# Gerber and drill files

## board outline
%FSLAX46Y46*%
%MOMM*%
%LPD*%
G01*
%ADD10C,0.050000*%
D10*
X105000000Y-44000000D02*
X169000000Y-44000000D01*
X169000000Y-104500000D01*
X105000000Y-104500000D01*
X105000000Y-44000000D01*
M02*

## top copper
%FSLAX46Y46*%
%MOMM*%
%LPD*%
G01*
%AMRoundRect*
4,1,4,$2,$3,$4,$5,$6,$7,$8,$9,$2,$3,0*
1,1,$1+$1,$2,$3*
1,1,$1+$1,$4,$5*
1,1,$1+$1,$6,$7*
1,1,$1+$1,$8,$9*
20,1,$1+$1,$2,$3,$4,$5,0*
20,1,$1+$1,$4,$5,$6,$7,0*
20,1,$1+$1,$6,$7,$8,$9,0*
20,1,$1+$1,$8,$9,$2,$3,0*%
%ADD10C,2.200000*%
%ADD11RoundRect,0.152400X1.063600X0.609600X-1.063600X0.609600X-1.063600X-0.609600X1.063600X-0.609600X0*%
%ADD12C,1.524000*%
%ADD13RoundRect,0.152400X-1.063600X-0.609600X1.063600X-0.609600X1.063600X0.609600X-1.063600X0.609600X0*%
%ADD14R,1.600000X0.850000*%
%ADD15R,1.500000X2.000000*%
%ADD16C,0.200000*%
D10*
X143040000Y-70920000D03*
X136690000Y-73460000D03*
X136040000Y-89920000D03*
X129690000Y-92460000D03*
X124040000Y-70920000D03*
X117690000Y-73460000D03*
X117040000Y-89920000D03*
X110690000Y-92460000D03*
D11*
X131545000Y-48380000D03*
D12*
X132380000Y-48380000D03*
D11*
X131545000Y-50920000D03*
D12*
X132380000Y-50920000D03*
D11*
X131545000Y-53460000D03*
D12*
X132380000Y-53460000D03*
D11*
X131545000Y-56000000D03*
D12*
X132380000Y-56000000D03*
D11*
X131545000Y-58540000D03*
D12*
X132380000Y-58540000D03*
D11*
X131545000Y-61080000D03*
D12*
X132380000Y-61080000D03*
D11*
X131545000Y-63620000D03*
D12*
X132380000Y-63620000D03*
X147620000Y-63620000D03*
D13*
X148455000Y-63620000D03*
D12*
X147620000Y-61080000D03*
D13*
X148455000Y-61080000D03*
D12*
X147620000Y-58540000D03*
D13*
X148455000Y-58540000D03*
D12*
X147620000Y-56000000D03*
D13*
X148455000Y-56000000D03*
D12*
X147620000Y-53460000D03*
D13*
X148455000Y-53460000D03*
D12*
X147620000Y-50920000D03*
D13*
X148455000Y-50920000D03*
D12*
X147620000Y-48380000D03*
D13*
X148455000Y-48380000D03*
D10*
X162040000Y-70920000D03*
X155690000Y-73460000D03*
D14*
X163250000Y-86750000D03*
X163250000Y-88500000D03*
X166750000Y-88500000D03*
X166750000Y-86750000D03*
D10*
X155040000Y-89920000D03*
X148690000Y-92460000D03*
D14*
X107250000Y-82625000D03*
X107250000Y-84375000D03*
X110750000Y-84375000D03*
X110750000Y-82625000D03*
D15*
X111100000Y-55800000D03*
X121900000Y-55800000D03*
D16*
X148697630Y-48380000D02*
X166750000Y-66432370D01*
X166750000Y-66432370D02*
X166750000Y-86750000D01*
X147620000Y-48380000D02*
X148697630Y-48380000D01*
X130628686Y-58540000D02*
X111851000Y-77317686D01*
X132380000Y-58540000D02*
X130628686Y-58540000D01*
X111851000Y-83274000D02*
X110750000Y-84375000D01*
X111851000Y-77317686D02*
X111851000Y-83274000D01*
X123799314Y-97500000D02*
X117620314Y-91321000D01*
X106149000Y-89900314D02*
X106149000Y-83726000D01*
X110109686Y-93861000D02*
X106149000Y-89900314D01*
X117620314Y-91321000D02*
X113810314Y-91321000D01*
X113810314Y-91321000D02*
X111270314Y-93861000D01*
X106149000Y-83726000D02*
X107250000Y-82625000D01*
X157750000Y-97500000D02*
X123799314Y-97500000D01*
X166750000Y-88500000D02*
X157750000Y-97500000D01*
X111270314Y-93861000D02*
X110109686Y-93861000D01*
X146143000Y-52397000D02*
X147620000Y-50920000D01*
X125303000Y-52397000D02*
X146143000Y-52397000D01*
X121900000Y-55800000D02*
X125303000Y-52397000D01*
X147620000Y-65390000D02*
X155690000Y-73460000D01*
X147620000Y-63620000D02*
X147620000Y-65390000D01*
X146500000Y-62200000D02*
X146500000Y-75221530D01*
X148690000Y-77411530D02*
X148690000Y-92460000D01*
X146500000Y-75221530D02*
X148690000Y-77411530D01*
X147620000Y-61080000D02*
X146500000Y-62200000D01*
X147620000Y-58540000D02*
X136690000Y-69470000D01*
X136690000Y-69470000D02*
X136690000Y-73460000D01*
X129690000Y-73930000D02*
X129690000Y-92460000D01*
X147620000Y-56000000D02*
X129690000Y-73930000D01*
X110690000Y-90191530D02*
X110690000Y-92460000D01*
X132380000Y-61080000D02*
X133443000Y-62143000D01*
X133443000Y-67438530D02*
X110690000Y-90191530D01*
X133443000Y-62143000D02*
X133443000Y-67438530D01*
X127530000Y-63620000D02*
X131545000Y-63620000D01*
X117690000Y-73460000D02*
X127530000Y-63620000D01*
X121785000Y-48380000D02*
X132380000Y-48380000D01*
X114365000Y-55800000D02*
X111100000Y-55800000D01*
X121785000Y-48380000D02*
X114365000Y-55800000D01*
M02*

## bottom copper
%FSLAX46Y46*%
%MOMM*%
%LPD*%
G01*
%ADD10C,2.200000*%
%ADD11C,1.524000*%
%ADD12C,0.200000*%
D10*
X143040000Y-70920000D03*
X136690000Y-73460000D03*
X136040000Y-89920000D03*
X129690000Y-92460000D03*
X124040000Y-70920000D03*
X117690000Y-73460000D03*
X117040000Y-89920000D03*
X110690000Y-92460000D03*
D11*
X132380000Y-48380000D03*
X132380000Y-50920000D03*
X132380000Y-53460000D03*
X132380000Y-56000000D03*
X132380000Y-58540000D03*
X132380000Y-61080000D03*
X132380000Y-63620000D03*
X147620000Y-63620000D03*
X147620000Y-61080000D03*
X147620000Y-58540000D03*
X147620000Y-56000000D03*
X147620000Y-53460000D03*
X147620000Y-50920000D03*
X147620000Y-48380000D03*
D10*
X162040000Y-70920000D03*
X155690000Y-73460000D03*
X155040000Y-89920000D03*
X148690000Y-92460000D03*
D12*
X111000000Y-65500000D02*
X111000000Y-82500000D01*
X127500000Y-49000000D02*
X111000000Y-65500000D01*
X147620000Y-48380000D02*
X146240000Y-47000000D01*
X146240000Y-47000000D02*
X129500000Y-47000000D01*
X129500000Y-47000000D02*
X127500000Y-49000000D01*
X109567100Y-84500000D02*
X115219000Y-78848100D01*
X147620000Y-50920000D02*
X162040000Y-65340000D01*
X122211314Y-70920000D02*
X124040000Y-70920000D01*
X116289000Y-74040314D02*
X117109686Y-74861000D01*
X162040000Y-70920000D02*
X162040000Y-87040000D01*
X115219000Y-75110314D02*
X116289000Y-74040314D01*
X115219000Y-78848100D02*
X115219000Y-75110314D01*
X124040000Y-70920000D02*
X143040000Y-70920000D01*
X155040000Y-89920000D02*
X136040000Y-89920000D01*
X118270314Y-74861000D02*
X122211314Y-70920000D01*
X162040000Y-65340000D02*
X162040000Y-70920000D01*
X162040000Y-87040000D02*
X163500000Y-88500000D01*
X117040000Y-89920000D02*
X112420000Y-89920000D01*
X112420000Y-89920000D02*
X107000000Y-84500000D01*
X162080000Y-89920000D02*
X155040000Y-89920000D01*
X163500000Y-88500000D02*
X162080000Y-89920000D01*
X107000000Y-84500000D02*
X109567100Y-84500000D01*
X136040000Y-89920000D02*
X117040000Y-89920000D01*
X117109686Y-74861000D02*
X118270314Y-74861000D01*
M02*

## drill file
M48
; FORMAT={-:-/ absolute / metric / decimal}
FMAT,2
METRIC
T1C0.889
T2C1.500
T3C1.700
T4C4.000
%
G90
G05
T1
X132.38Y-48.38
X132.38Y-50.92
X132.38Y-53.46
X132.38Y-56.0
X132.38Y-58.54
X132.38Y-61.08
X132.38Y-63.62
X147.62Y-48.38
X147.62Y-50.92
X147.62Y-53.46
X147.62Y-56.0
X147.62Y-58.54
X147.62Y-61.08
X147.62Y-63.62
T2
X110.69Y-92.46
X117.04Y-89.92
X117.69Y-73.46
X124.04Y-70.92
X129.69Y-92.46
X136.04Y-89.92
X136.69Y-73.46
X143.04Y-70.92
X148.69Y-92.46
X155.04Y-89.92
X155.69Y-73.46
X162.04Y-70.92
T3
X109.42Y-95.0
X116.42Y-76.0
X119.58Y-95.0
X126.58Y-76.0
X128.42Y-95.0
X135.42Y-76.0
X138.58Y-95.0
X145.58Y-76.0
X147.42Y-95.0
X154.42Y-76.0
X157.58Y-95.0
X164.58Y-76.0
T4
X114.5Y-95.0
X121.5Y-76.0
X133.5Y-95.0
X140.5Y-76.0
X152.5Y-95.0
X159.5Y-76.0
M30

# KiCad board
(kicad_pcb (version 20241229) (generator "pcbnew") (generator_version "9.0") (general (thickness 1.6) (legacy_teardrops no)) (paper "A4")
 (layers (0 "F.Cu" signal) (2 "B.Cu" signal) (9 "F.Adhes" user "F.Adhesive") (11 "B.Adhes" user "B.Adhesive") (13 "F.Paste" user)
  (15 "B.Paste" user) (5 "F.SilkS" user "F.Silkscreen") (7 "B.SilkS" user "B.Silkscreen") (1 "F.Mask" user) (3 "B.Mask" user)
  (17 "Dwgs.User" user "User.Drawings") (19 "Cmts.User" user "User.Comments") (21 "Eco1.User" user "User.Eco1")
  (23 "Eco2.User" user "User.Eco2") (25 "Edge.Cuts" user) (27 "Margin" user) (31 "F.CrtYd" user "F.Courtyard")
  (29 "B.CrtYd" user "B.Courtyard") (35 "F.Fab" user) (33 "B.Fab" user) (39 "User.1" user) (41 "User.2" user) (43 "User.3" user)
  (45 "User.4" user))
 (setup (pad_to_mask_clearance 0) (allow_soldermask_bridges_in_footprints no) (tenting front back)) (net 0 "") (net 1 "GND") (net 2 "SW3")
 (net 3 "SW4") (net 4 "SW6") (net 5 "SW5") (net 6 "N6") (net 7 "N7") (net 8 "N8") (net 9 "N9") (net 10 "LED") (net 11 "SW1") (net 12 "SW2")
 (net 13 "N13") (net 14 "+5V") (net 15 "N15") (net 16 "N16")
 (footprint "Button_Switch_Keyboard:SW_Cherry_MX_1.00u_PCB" (layer "F.Cu") (at 143.04 70.92)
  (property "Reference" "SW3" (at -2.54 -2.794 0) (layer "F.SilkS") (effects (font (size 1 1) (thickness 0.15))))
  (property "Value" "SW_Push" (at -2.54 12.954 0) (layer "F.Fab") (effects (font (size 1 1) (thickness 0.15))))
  (pad "" np_thru_hole circle (at -7.62 5.08) (size 1.7 1.7) (drill 1.7) (layers "*.Cu" "*.Mask"))
  (pad "" np_thru_hole circle (at -2.54 5.08) (size 4 4) (drill 4) (layers "*.Cu" "*.Mask"))
  (pad "" np_thru_hole circle (at 2.54 5.08) (size 1.7 1.7) (drill 1.7) (layers "*.Cu" "*.Mask"))
  (pad "1" thru_hole circle (at 0 0) (size 2.2 2.2) (drill 1.5) (layers "*.Cu" "*.Mask") (remove_unused_layers no) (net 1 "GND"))
  (pad "2" thru_hole circle (at -6.35 2.54) (size 2.2 2.2) (drill 1.5) (layers "*.Cu" "*.Mask") (remove_unused_layers no) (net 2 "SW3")))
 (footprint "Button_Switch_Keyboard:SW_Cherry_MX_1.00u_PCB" (layer "F.Cu") (at 136.04 89.92)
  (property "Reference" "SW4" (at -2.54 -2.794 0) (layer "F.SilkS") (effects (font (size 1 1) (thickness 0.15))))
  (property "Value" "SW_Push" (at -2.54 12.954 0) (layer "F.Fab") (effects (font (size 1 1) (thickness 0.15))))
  (pad "" np_thru_hole circle (at -7.62 5.08) (size 1.7 1.7) (drill 1.7) (layers "*.Cu" "*.Mask"))
  (pad "" np_thru_hole circle (at -2.54 5.08) (size 4 4) (drill 4) (layers "*.Cu" "*.Mask"))
  (pad "" np_thru_hole circle (at 2.54 5.08) (size 1.7 1.7) (drill 1.7) (layers "*.Cu" "*.Mask"))
  (pad "1" thru_hole circle (at 0 0) (size 2.2 2.2) (drill 1.5) (layers "*.Cu" "*.Mask") (remove_unused_layers no) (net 1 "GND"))
  (pad "2" thru_hole circle (at -6.35 2.54) (size 2.2 2.2) (drill 1.5) (layers "*.Cu" "*.Mask") (remove_unused_layers no) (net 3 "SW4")))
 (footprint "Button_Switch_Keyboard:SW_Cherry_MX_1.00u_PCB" (layer "F.Cu") (at 124.04 70.92)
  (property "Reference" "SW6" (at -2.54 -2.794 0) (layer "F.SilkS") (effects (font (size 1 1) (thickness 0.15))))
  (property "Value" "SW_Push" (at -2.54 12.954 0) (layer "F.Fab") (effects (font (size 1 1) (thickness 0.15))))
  (pad "" np_thru_hole circle (at -7.62 5.08) (size 1.7 1.7) (drill 1.7) (layers "*.Cu" "*.Mask"))
  (pad "" np_thru_hole circle (at -2.54 5.08) (size 4 4) (drill 4) (layers "*.Cu" "*.Mask"))
  (pad "" np_thru_hole circle (at 2.54 5.08) (size 1.7 1.7) (drill 1.7) (layers "*.Cu" "*.Mask"))
  (pad "1" thru_hole circle (at 0 0) (size 2.2 2.2) (drill 1.5) (layers "*.Cu" "*.Mask") (remove_unused_layers no) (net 1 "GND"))
  (pad "2" thru_hole circle (at -6.35 2.54) (size 2.2 2.2) (drill 1.5) (layers "*.Cu" "*.Mask") (remove_unused_layers no) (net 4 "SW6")))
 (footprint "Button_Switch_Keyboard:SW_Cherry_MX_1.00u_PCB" (layer "F.Cu") (at 117.04 89.92)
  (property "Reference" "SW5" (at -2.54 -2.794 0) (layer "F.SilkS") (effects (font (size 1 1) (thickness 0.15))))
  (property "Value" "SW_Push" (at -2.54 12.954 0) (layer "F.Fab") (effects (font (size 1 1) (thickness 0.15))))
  (pad "" np_thru_hole circle (at -7.62 5.08) (size 1.7 1.7) (drill 1.7) (layers "*.Cu" "*.Mask"))
  (pad "" np_thru_hole circle (at -2.54 5.08) (size 4 4) (drill 4) (layers "*.Cu" "*.Mask"))
  (pad "" np_thru_hole circle (at 2.54 5.08) (size 1.7 1.7) (drill 1.7) (layers "*.Cu" "*.Mask"))
  (pad "1" thru_hole circle (at 0 0) (size 2.2 2.2) (drill 1.5) (layers "*.Cu" "*.Mask") (remove_unused_layers no) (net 1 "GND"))
  (pad "2" thru_hole circle (at -6.35 2.54) (size 2.2 2.2) (drill 1.5) (layers "*.Cu" "*.Mask") (remove_unused_layers no) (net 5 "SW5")))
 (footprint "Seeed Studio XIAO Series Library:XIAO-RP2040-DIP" (layer "F.Cu") (at 140 56)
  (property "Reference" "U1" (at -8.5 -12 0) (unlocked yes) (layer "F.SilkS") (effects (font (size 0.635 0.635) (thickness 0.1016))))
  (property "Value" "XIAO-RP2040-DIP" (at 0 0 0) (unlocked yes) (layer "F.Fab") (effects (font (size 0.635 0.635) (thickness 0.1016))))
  (pad "1" smd roundrect (at -8.455 -7.62 180) (size 2.432 1.524) (layers "F.Cu" "F.Mask") (roundrect_rratio 0.1) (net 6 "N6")
   (thermal_bridge_angle 45))
  (pad "1" thru_hole circle (at -7.62 -7.62 180) (size 1.524 1.524) (drill 0.889) (layers "*.Cu" "*.Mask") (remove_unused_layers no)
   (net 6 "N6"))
  (pad "2" smd roundrect (at -8.455 -5.08 180) (size 2.432 1.524) (layers "F.Cu" "F.Mask") (roundrect_rratio 0.1) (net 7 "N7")
   (thermal_bridge_angle 45))
  (pad "2" thru_hole circle (at -7.62 -5.08 180) (size 1.524 1.524) (drill 0.889) (layers "*.Cu" "*.Mask") (remove_unused_layers no)
   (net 7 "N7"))
  (pad "3" smd roundrect (at -8.455 -2.54 180) (size 2.432 1.524) (layers "F.Cu" "F.Mask") (roundrect_rratio 0.1) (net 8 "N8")
   (thermal_bridge_angle 45))
  (pad "3" thru_hole circle (at -7.62 -2.54 180) (size 1.524 1.524) (drill 0.889) (layers "*.Cu" "*.Mask") (remove_unused_layers no)
   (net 8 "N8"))
  (pad "4" smd roundrect (at -8.455 0 180) (size 2.432 1.524) (layers "F.Cu" "F.Mask") (roundrect_rratio 0.1) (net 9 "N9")
   (thermal_bridge_angle 45))
  (pad "4" thru_hole circle (at -7.62 0 180) (size 1.524 1.524) (drill 0.889) (layers "*.Cu" "*.Mask") (remove_unused_layers no)
   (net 9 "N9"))
  (pad "5" smd roundrect (at -8.455 2.54 180) (size 2.432 1.524) (layers "F.Cu" "F.Mask") (roundrect_rratio 0.1) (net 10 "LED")
   (thermal_bridge_angle 45))
  (pad "5" thru_hole circle (at -7.62 2.54 180) (size 1.524 1.524) (drill 0.889) (layers "*.Cu" "*.Mask") (remove_unused_layers no)
   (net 10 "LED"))
  (pad "6" smd roundrect (at -8.455 5.08 180) (size 2.432 1.524) (layers "F.Cu" "F.Mask") (roundrect_rratio 0.1) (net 5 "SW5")
   (thermal_bridge_angle 45))
  (pad "6" thru_hole circle (at -7.62 5.08 180) (size 1.524 1.524) (drill 0.889) (layers "*.Cu" "*.Mask") (remove_unused_layers no)
   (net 5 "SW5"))
  (pad "7" smd roundrect (at -8.455 7.62 180) (size 2.432 1.524) (layers "F.Cu" "F.Mask") (roundrect_rratio 0.1) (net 4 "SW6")
   (thermal_bridge_angle 45))
  (pad "7" thru_hole circle (at -7.62 7.62 180) (size 1.524 1.524) (drill 0.889) (layers "*.Cu" "*.Mask") (remove_unused_layers no)
   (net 4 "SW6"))
  (pad "8" thru_hole circle (at 7.62 7.62) (size 1.524 1.524) (drill 0.889) (layers "*.Cu" "*.Mask") (remove_unused_layers no)
   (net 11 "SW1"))
  (pad "8" smd roundrect (at 8.455 7.62) (size 2.432 1.524) (layers "F.Cu" "F.Mask") (roundrect_rratio 0.1) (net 11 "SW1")
   (thermal_bridge_angle 45))
  (pad "9" thru_hole circle (at 7.62 5.08) (size 1.524 1.524) (drill 0.889) (layers "*.Cu" "*.Mask") (remove_unused_layers no)
   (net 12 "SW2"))
  (pad "9" smd roundrect (at 8.455 5.08) (size 2.432 1.524) (layers "F.Cu" "F.Mask") (roundrect_rratio 0.1) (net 12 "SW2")
   (thermal_bridge_angle 45))
  (pad "10" thru_hole circle (at 7.62 2.54) (size 1.524 1.524) (drill 0.889) (layers "*.Cu" "*.Mask") (remove_unused_layers no)
   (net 2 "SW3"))
  (pad "10" smd roundrect (at 8.455 2.54) (size 2.432 1.524) (layers "F.Cu" "F.Mask") (roundrect_rratio 0.1) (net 2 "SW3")
   (thermal_bridge_angle 45))
  (pad "11" thru_hole circle (at 7.62 0) (size 1.524 1.524) (drill 0.889) (layers "*.Cu" "*.Mask") (remove_unused_layers no) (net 3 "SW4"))
  (pad "11" smd roundrect (at 8.455 0) (size 2.432 1.524) (layers "F.Cu" "F.Mask") (roundrect_rratio 0.1) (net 3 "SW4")
   (thermal_bridge_angle 45))
  (pad "12" thru_hole circle (at 7.62 -2.54) (size 1.524 1.524) (drill 0.889) (layers "*.Cu" "*.Mask") (remove_unused_layers no)
   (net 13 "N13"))
  (pad "12" smd roundrect (at 8.455 -2.54) (size 2.432 1.524) (layers "F.Cu" "F.Mask") (roundrect_rratio 0.1) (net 13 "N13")
   (thermal_bridge_angle 45))
  (pad "13" thru_hole circle (at 7.62 -5.08) (size 1.524 1.524) (drill 0.889) (layers "*.Cu" "*.Mask") (remove_unused_layers no)
   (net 1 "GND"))
  (pad "13" smd roundrect (at 8.455 -5.08) (size 2.432 1.524) (layers "F.Cu" "F.Mask") (roundrect_rratio 0.1) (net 1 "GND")
   (thermal_bridge_angle 45))
  (pad "14" thru_hole circle (at 7.62 -7.62) (size 1.524 1.524) (drill 0.889) (layers "*.Cu" "*.Mask") (remove_unused_layers no)
   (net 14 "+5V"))
  (pad "14" smd roundrect (at 8.455 -7.62) (size 2.432 1.524) (layers "F.Cu" "F.Mask") (roundrect_rratio 0.1) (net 14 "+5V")
   (thermal_bridge_angle 45)))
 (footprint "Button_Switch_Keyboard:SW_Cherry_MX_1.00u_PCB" (layer "F.Cu") (at 162.04 70.92)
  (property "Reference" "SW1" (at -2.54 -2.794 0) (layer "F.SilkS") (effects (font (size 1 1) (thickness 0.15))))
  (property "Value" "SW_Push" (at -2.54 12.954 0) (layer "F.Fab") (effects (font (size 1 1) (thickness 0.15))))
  (pad "" np_thru_hole circle (at -7.62 5.08) (size 1.7 1.7) (drill 1.7) (layers "*.Cu" "*.Mask"))
  (pad "" np_thru_hole circle (at -2.54 5.08) (size 4 4) (drill 4) (layers "*.Cu" "*.Mask"))
  (pad "" np_thru_hole circle (at 2.54 5.08) (size 1.7 1.7) (drill 1.7) (layers "*.Cu" "*.Mask"))
  (pad "1" thru_hole circle (at 0 0) (size 2.2 2.2) (drill 1.5) (layers "*.Cu" "*.Mask") (remove_unused_layers no) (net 1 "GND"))
  (pad "2" thru_hole circle (at -6.35 2.54) (size 2.2 2.2) (drill 1.5) (layers "*.Cu" "*.Mask") (remove_unused_layers no) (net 11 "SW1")))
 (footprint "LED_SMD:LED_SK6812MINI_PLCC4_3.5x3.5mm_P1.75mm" (layer "F.Cu") (at 165 87.625)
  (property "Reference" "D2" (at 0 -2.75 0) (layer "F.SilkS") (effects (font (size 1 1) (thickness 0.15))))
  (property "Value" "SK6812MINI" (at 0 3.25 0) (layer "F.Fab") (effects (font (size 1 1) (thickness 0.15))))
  (pad "1" smd rect (at -1.75 -0.875) (size 1.6 0.85) (layers "F.Cu" "F.Mask" "F.Paste") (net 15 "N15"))
  (pad "2" smd rect (at -1.75 0.875) (size 1.6 0.85) (layers "F.Cu" "F.Mask" "F.Paste") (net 1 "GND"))
  (pad "3" smd rect (at 1.75 0.875) (size 1.6 0.85) (layers "F.Cu" "F.Mask" "F.Paste") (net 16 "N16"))
  (pad "4" smd rect (at 1.75 -0.875) (size 1.6 0.85) (layers "F.Cu" "F.Mask" "F.Paste") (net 14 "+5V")))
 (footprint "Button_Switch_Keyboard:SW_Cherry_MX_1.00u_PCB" (layer "F.Cu") (at 155.04 89.92)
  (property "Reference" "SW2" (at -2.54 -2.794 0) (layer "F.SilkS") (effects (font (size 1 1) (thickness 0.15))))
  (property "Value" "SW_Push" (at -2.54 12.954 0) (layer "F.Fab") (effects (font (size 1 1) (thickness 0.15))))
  (pad "" np_thru_hole circle (at -7.62 5.08) (size 1.7 1.7) (drill 1.7) (layers "*.Cu" "*.Mask"))
  (pad "" np_thru_hole circle (at -2.54 5.08) (size 4 4) (drill 4) (layers "*.Cu" "*.Mask"))
  (pad "" np_thru_hole circle (at 2.54 5.08) (size 1.7 1.7) (drill 1.7) (layers "*.Cu" "*.Mask"))
  (pad "1" thru_hole circle (at 0 0) (size 2.2 2.2) (drill 1.5) (layers "*.Cu" "*.Mask") (remove_unused_layers no) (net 1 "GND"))
  (pad "2" thru_hole circle (at -6.35 2.54) (size 2.2 2.2) (drill 1.5) (layers "*.Cu" "*.Mask") (remove_unused_layers no) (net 12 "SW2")))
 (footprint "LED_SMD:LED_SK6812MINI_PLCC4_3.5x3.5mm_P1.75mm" (layer "F.Cu") (at 109 83.5)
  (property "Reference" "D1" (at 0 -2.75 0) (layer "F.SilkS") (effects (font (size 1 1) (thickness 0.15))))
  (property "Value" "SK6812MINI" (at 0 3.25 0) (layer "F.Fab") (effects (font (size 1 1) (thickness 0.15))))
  (pad "1" smd rect (at -1.75 -0.875) (size 1.6 0.85) (layers "F.Cu" "F.Mask" "F.Paste") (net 16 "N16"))
  (pad "2" smd rect (at -1.75 0.875) (size 1.6 0.85) (layers "F.Cu" "F.Mask" "F.Paste") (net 1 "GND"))
  (pad "3" smd rect (at 1.75 0.875) (size 1.6 0.85) (layers "F.Cu" "F.Mask" "F.Paste") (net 10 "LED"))
  (pad "4" smd rect (at 1.75 -0.875) (size 1.6 0.85) (layers "F.Cu" "F.Mask" "F.Paste") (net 14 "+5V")))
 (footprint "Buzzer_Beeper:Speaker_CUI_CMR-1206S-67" (layer "F.Cu") (at 116.5 53.5)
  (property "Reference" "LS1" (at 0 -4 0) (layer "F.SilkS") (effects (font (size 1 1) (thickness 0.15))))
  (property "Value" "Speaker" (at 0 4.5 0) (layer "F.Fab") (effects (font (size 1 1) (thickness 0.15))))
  (pad "1" smd rect (at -5.4 2.3 180) (size 1.5 2) (layers "F.Cu" "F.Mask") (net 6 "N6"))
  (pad "2" smd rect (at 5.4 2.3 180) (size 1.5 2) (layers "F.Cu" "F.Mask") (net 1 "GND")))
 (gr_rect (start 105 44) (end 169 104.5) (stroke (width 0.05) (type default)) (fill no) (layer "Edge.Cuts"))
 (segment (start 148.69763 48.38) (end 166.75 66.43237) (width 0.2) (layer "F.Cu") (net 14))
 (segment (start 166.75 66.43237) (end 166.75 86.75) (width 0.2) (layer "F.Cu") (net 14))
 (segment (start 147.62 48.38) (end 148.69763 48.38) (width 0.2) (layer "F.Cu") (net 14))
 (segment (start 111 65.5) (end 111 82.5) (width 0.2) (layer "B.Cu") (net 14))
 (segment (start 127.5 49) (end 111 65.5) (width 0.2) (layer "B.Cu") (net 14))
 (segment (start 147.62 48.38) (end 146.24 47) (width 0.2) (layer "B.Cu") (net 14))
 (segment (start 146.24 47) (end 129.5 47) (width 0.2) (layer "B.Cu") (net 14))
 (segment (start 129.5 47) (end 127.5 49) (width 0.2) (layer "B.Cu") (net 14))
 (segment (start 130.628686 58.54) (end 111.851 77.317686) (width 0.2) (layer "F.Cu") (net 10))
 (segment (start 132.38 58.54) (end 130.628686 58.54) (width 0.2) (layer "F.Cu") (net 10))
 (segment (start 111.851 83.274) (end 110.75 84.375) (width 0.2) (layer "F.Cu") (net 10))
 (segment (start 111.851 77.317686) (end 111.851 83.274) (width 0.2) (layer "F.Cu") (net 10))
 (segment (start 123.799314 97.5) (end 117.620314 91.321) (width 0.2) (layer "F.Cu") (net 16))
 (segment (start 106.149 89.900314) (end 106.149 83.726) (width 0.2) (layer "F.Cu") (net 16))
 (segment (start 110.109686 93.861) (end 106.149 89.900314) (width 0.2) (layer "F.Cu") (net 16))
 (segment (start 117.620314 91.321) (end 113.810314 91.321) (width 0.2) (layer "F.Cu") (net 16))
 (segment (start 113.810314 91.321) (end 111.270314 93.861) (width 0.2) (layer "F.Cu") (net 16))
 (segment (start 106.149 83.726) (end 107.25 82.625) (width 0.2) (layer "F.Cu") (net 16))
 (segment (start 157.75 97.5) (end 123.799314 97.5) (width 0.2) (layer "F.Cu") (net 16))
 (segment (start 166.75 88.5) (end 157.75 97.5) (width 0.2) (layer "F.Cu") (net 16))
 (segment (start 111.270314 93.861) (end 110.109686 93.861) (width 0.2) (layer "F.Cu") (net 16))
 (segment (start 146.143 52.397) (end 147.62 50.92) (width 0.2) (layer "F.Cu") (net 1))
 (segment (start 125.303 52.397) (end 146.143 52.397) (width 0.2) (layer "F.Cu") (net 1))
 (segment (start 121.9 55.8) (end 125.303 52.397) (width 0.2) (layer "F.Cu") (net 1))
 (segment (start 109.5671 84.5) (end 115.219 78.8481) (width 0.2) (layer "B.Cu") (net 1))
 (segment (start 147.62 50.92) (end 162.04 65.34) (width 0.2) (layer "B.Cu") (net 1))
 (segment (start 122.211314 70.92) (end 124.04 70.92) (width 0.2) (layer "B.Cu") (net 1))
 (segment (start 116.289 74.040314) (end 117.109686 74.861) (width 0.2) (layer "B.Cu") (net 1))
 (segment (start 162.04 70.92) (end 162.04 87.04) (width 0.2) (layer "B.Cu") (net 1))
 (segment (start 115.219 75.110314) (end 116.289 74.040314) (width 0.2) (layer "B.Cu") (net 1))
 (segment (start 115.219 78.8481) (end 115.219 75.110314) (width 0.2) (layer "B.Cu") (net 1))
 (segment (start 124.04 70.92) (end 143.04 70.92) (width 0.2) (layer "B.Cu") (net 1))
 (segment (start 155.04 89.92) (end 136.04 89.92) (width 0.2) (layer "B.Cu") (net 1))
 (segment (start 118.270314 74.861) (end 122.211314 70.92) (width 0.2) (layer "B.Cu") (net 1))
 (segment (start 162.04 65.34) (end 162.04 70.92) (width 0.2) (layer "B.Cu") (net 1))
 (segment (start 162.04 87.04) (end 163.5 88.5) (width 0.2) (layer "B.Cu") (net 1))
 (segment (start 117.04 89.92) (end 112.42 89.92) (width 0.2) (layer "B.Cu") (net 1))
 (segment (start 112.42 89.92) (end 107 84.5) (width 0.2) (layer "B.Cu") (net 1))
 (segment (start 162.08 89.92) (end 155.04 89.92) (width 0.2) (layer "B.Cu") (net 1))
 (segment (start 163.5 88.5) (end 162.08 89.92) (width 0.2) (layer "B.Cu") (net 1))
 (segment (start 107 84.5) (end 109.5671 84.5) (width 0.2) (layer "B.Cu") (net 1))
 (segment (start 136.04 89.92) (end 117.04 89.92) (width 0.2) (layer "B.Cu") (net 1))
 (segment (start 117.109686 74.861) (end 118.270314 74.861) (width 0.2) (layer "B.Cu") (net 1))
 (segment (start 147.62 65.39) (end 155.69 73.46) (width 0.2) (layer "F.Cu") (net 11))
 (segment (start 147.62 63.62) (end 147.62 65.39) (width 0.2) (layer "F.Cu") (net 11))
 (segment (start 146.5 62.2) (end 146.5 75.22153) (width 0.2) (layer "F.Cu") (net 12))
 (segment (start 148.69 77.41153) (end 148.69 92.46) (width 0.2) (layer "F.Cu") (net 12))
 (segment (start 146.5 75.22153) (end 148.69 77.41153) (width 0.2) (layer "F.Cu") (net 12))
 (segment (start 147.62 61.08) (end 146.5 62.2) (width 0.2) (layer "F.Cu") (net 12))
 (segment (start 147.62 58.54) (end 136.69 69.47) (width 0.2) (layer "F.Cu") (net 2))
 (segment (start 136.69 69.47) (end 136.69 73.46) (width 0.2) (layer "F.Cu") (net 2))
 (segment (start 129.69 73.93) (end 129.69 92.46) (width 0.2) (layer "F.Cu") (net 3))
 (segment (start 147.62 56) (end 129.69 73.93) (width 0.2) (layer "F.Cu") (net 3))
 (segment (start 110.69 90.19153) (end 110.69 92.46) (width 0.2) (layer "F.Cu") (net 5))
 (segment (start 132.38 61.08) (end 133.443 62.143) (width 0.2) (layer "F.Cu") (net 5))
 (segment (start 133.443 67.43853) (end 110.69 90.19153) (width 0.2) (layer "F.Cu") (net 5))
 (segment (start 133.443 62.143) (end 133.443 67.43853) (width 0.2) (layer "F.Cu") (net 5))
 (segment (start 127.53 63.62) (end 131.545 63.62) (width 0.2) (layer "F.Cu") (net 4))
 (segment (start 117.69 73.46) (end 127.53 63.62) (width 0.2) (layer "F.Cu") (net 4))
 (segment (start 121.785 48.38) (end 132.38 48.38) (width 0.2) (layer "F.Cu") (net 6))
 (segment (start 114.365 55.8) (end 111.1 55.8) (width 0.2) (layer "F.Cu") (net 6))
 (segment (start 121.785 48.38) (end 114.365 55.8) (width 0.2) (layer "F.Cu") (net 6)))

